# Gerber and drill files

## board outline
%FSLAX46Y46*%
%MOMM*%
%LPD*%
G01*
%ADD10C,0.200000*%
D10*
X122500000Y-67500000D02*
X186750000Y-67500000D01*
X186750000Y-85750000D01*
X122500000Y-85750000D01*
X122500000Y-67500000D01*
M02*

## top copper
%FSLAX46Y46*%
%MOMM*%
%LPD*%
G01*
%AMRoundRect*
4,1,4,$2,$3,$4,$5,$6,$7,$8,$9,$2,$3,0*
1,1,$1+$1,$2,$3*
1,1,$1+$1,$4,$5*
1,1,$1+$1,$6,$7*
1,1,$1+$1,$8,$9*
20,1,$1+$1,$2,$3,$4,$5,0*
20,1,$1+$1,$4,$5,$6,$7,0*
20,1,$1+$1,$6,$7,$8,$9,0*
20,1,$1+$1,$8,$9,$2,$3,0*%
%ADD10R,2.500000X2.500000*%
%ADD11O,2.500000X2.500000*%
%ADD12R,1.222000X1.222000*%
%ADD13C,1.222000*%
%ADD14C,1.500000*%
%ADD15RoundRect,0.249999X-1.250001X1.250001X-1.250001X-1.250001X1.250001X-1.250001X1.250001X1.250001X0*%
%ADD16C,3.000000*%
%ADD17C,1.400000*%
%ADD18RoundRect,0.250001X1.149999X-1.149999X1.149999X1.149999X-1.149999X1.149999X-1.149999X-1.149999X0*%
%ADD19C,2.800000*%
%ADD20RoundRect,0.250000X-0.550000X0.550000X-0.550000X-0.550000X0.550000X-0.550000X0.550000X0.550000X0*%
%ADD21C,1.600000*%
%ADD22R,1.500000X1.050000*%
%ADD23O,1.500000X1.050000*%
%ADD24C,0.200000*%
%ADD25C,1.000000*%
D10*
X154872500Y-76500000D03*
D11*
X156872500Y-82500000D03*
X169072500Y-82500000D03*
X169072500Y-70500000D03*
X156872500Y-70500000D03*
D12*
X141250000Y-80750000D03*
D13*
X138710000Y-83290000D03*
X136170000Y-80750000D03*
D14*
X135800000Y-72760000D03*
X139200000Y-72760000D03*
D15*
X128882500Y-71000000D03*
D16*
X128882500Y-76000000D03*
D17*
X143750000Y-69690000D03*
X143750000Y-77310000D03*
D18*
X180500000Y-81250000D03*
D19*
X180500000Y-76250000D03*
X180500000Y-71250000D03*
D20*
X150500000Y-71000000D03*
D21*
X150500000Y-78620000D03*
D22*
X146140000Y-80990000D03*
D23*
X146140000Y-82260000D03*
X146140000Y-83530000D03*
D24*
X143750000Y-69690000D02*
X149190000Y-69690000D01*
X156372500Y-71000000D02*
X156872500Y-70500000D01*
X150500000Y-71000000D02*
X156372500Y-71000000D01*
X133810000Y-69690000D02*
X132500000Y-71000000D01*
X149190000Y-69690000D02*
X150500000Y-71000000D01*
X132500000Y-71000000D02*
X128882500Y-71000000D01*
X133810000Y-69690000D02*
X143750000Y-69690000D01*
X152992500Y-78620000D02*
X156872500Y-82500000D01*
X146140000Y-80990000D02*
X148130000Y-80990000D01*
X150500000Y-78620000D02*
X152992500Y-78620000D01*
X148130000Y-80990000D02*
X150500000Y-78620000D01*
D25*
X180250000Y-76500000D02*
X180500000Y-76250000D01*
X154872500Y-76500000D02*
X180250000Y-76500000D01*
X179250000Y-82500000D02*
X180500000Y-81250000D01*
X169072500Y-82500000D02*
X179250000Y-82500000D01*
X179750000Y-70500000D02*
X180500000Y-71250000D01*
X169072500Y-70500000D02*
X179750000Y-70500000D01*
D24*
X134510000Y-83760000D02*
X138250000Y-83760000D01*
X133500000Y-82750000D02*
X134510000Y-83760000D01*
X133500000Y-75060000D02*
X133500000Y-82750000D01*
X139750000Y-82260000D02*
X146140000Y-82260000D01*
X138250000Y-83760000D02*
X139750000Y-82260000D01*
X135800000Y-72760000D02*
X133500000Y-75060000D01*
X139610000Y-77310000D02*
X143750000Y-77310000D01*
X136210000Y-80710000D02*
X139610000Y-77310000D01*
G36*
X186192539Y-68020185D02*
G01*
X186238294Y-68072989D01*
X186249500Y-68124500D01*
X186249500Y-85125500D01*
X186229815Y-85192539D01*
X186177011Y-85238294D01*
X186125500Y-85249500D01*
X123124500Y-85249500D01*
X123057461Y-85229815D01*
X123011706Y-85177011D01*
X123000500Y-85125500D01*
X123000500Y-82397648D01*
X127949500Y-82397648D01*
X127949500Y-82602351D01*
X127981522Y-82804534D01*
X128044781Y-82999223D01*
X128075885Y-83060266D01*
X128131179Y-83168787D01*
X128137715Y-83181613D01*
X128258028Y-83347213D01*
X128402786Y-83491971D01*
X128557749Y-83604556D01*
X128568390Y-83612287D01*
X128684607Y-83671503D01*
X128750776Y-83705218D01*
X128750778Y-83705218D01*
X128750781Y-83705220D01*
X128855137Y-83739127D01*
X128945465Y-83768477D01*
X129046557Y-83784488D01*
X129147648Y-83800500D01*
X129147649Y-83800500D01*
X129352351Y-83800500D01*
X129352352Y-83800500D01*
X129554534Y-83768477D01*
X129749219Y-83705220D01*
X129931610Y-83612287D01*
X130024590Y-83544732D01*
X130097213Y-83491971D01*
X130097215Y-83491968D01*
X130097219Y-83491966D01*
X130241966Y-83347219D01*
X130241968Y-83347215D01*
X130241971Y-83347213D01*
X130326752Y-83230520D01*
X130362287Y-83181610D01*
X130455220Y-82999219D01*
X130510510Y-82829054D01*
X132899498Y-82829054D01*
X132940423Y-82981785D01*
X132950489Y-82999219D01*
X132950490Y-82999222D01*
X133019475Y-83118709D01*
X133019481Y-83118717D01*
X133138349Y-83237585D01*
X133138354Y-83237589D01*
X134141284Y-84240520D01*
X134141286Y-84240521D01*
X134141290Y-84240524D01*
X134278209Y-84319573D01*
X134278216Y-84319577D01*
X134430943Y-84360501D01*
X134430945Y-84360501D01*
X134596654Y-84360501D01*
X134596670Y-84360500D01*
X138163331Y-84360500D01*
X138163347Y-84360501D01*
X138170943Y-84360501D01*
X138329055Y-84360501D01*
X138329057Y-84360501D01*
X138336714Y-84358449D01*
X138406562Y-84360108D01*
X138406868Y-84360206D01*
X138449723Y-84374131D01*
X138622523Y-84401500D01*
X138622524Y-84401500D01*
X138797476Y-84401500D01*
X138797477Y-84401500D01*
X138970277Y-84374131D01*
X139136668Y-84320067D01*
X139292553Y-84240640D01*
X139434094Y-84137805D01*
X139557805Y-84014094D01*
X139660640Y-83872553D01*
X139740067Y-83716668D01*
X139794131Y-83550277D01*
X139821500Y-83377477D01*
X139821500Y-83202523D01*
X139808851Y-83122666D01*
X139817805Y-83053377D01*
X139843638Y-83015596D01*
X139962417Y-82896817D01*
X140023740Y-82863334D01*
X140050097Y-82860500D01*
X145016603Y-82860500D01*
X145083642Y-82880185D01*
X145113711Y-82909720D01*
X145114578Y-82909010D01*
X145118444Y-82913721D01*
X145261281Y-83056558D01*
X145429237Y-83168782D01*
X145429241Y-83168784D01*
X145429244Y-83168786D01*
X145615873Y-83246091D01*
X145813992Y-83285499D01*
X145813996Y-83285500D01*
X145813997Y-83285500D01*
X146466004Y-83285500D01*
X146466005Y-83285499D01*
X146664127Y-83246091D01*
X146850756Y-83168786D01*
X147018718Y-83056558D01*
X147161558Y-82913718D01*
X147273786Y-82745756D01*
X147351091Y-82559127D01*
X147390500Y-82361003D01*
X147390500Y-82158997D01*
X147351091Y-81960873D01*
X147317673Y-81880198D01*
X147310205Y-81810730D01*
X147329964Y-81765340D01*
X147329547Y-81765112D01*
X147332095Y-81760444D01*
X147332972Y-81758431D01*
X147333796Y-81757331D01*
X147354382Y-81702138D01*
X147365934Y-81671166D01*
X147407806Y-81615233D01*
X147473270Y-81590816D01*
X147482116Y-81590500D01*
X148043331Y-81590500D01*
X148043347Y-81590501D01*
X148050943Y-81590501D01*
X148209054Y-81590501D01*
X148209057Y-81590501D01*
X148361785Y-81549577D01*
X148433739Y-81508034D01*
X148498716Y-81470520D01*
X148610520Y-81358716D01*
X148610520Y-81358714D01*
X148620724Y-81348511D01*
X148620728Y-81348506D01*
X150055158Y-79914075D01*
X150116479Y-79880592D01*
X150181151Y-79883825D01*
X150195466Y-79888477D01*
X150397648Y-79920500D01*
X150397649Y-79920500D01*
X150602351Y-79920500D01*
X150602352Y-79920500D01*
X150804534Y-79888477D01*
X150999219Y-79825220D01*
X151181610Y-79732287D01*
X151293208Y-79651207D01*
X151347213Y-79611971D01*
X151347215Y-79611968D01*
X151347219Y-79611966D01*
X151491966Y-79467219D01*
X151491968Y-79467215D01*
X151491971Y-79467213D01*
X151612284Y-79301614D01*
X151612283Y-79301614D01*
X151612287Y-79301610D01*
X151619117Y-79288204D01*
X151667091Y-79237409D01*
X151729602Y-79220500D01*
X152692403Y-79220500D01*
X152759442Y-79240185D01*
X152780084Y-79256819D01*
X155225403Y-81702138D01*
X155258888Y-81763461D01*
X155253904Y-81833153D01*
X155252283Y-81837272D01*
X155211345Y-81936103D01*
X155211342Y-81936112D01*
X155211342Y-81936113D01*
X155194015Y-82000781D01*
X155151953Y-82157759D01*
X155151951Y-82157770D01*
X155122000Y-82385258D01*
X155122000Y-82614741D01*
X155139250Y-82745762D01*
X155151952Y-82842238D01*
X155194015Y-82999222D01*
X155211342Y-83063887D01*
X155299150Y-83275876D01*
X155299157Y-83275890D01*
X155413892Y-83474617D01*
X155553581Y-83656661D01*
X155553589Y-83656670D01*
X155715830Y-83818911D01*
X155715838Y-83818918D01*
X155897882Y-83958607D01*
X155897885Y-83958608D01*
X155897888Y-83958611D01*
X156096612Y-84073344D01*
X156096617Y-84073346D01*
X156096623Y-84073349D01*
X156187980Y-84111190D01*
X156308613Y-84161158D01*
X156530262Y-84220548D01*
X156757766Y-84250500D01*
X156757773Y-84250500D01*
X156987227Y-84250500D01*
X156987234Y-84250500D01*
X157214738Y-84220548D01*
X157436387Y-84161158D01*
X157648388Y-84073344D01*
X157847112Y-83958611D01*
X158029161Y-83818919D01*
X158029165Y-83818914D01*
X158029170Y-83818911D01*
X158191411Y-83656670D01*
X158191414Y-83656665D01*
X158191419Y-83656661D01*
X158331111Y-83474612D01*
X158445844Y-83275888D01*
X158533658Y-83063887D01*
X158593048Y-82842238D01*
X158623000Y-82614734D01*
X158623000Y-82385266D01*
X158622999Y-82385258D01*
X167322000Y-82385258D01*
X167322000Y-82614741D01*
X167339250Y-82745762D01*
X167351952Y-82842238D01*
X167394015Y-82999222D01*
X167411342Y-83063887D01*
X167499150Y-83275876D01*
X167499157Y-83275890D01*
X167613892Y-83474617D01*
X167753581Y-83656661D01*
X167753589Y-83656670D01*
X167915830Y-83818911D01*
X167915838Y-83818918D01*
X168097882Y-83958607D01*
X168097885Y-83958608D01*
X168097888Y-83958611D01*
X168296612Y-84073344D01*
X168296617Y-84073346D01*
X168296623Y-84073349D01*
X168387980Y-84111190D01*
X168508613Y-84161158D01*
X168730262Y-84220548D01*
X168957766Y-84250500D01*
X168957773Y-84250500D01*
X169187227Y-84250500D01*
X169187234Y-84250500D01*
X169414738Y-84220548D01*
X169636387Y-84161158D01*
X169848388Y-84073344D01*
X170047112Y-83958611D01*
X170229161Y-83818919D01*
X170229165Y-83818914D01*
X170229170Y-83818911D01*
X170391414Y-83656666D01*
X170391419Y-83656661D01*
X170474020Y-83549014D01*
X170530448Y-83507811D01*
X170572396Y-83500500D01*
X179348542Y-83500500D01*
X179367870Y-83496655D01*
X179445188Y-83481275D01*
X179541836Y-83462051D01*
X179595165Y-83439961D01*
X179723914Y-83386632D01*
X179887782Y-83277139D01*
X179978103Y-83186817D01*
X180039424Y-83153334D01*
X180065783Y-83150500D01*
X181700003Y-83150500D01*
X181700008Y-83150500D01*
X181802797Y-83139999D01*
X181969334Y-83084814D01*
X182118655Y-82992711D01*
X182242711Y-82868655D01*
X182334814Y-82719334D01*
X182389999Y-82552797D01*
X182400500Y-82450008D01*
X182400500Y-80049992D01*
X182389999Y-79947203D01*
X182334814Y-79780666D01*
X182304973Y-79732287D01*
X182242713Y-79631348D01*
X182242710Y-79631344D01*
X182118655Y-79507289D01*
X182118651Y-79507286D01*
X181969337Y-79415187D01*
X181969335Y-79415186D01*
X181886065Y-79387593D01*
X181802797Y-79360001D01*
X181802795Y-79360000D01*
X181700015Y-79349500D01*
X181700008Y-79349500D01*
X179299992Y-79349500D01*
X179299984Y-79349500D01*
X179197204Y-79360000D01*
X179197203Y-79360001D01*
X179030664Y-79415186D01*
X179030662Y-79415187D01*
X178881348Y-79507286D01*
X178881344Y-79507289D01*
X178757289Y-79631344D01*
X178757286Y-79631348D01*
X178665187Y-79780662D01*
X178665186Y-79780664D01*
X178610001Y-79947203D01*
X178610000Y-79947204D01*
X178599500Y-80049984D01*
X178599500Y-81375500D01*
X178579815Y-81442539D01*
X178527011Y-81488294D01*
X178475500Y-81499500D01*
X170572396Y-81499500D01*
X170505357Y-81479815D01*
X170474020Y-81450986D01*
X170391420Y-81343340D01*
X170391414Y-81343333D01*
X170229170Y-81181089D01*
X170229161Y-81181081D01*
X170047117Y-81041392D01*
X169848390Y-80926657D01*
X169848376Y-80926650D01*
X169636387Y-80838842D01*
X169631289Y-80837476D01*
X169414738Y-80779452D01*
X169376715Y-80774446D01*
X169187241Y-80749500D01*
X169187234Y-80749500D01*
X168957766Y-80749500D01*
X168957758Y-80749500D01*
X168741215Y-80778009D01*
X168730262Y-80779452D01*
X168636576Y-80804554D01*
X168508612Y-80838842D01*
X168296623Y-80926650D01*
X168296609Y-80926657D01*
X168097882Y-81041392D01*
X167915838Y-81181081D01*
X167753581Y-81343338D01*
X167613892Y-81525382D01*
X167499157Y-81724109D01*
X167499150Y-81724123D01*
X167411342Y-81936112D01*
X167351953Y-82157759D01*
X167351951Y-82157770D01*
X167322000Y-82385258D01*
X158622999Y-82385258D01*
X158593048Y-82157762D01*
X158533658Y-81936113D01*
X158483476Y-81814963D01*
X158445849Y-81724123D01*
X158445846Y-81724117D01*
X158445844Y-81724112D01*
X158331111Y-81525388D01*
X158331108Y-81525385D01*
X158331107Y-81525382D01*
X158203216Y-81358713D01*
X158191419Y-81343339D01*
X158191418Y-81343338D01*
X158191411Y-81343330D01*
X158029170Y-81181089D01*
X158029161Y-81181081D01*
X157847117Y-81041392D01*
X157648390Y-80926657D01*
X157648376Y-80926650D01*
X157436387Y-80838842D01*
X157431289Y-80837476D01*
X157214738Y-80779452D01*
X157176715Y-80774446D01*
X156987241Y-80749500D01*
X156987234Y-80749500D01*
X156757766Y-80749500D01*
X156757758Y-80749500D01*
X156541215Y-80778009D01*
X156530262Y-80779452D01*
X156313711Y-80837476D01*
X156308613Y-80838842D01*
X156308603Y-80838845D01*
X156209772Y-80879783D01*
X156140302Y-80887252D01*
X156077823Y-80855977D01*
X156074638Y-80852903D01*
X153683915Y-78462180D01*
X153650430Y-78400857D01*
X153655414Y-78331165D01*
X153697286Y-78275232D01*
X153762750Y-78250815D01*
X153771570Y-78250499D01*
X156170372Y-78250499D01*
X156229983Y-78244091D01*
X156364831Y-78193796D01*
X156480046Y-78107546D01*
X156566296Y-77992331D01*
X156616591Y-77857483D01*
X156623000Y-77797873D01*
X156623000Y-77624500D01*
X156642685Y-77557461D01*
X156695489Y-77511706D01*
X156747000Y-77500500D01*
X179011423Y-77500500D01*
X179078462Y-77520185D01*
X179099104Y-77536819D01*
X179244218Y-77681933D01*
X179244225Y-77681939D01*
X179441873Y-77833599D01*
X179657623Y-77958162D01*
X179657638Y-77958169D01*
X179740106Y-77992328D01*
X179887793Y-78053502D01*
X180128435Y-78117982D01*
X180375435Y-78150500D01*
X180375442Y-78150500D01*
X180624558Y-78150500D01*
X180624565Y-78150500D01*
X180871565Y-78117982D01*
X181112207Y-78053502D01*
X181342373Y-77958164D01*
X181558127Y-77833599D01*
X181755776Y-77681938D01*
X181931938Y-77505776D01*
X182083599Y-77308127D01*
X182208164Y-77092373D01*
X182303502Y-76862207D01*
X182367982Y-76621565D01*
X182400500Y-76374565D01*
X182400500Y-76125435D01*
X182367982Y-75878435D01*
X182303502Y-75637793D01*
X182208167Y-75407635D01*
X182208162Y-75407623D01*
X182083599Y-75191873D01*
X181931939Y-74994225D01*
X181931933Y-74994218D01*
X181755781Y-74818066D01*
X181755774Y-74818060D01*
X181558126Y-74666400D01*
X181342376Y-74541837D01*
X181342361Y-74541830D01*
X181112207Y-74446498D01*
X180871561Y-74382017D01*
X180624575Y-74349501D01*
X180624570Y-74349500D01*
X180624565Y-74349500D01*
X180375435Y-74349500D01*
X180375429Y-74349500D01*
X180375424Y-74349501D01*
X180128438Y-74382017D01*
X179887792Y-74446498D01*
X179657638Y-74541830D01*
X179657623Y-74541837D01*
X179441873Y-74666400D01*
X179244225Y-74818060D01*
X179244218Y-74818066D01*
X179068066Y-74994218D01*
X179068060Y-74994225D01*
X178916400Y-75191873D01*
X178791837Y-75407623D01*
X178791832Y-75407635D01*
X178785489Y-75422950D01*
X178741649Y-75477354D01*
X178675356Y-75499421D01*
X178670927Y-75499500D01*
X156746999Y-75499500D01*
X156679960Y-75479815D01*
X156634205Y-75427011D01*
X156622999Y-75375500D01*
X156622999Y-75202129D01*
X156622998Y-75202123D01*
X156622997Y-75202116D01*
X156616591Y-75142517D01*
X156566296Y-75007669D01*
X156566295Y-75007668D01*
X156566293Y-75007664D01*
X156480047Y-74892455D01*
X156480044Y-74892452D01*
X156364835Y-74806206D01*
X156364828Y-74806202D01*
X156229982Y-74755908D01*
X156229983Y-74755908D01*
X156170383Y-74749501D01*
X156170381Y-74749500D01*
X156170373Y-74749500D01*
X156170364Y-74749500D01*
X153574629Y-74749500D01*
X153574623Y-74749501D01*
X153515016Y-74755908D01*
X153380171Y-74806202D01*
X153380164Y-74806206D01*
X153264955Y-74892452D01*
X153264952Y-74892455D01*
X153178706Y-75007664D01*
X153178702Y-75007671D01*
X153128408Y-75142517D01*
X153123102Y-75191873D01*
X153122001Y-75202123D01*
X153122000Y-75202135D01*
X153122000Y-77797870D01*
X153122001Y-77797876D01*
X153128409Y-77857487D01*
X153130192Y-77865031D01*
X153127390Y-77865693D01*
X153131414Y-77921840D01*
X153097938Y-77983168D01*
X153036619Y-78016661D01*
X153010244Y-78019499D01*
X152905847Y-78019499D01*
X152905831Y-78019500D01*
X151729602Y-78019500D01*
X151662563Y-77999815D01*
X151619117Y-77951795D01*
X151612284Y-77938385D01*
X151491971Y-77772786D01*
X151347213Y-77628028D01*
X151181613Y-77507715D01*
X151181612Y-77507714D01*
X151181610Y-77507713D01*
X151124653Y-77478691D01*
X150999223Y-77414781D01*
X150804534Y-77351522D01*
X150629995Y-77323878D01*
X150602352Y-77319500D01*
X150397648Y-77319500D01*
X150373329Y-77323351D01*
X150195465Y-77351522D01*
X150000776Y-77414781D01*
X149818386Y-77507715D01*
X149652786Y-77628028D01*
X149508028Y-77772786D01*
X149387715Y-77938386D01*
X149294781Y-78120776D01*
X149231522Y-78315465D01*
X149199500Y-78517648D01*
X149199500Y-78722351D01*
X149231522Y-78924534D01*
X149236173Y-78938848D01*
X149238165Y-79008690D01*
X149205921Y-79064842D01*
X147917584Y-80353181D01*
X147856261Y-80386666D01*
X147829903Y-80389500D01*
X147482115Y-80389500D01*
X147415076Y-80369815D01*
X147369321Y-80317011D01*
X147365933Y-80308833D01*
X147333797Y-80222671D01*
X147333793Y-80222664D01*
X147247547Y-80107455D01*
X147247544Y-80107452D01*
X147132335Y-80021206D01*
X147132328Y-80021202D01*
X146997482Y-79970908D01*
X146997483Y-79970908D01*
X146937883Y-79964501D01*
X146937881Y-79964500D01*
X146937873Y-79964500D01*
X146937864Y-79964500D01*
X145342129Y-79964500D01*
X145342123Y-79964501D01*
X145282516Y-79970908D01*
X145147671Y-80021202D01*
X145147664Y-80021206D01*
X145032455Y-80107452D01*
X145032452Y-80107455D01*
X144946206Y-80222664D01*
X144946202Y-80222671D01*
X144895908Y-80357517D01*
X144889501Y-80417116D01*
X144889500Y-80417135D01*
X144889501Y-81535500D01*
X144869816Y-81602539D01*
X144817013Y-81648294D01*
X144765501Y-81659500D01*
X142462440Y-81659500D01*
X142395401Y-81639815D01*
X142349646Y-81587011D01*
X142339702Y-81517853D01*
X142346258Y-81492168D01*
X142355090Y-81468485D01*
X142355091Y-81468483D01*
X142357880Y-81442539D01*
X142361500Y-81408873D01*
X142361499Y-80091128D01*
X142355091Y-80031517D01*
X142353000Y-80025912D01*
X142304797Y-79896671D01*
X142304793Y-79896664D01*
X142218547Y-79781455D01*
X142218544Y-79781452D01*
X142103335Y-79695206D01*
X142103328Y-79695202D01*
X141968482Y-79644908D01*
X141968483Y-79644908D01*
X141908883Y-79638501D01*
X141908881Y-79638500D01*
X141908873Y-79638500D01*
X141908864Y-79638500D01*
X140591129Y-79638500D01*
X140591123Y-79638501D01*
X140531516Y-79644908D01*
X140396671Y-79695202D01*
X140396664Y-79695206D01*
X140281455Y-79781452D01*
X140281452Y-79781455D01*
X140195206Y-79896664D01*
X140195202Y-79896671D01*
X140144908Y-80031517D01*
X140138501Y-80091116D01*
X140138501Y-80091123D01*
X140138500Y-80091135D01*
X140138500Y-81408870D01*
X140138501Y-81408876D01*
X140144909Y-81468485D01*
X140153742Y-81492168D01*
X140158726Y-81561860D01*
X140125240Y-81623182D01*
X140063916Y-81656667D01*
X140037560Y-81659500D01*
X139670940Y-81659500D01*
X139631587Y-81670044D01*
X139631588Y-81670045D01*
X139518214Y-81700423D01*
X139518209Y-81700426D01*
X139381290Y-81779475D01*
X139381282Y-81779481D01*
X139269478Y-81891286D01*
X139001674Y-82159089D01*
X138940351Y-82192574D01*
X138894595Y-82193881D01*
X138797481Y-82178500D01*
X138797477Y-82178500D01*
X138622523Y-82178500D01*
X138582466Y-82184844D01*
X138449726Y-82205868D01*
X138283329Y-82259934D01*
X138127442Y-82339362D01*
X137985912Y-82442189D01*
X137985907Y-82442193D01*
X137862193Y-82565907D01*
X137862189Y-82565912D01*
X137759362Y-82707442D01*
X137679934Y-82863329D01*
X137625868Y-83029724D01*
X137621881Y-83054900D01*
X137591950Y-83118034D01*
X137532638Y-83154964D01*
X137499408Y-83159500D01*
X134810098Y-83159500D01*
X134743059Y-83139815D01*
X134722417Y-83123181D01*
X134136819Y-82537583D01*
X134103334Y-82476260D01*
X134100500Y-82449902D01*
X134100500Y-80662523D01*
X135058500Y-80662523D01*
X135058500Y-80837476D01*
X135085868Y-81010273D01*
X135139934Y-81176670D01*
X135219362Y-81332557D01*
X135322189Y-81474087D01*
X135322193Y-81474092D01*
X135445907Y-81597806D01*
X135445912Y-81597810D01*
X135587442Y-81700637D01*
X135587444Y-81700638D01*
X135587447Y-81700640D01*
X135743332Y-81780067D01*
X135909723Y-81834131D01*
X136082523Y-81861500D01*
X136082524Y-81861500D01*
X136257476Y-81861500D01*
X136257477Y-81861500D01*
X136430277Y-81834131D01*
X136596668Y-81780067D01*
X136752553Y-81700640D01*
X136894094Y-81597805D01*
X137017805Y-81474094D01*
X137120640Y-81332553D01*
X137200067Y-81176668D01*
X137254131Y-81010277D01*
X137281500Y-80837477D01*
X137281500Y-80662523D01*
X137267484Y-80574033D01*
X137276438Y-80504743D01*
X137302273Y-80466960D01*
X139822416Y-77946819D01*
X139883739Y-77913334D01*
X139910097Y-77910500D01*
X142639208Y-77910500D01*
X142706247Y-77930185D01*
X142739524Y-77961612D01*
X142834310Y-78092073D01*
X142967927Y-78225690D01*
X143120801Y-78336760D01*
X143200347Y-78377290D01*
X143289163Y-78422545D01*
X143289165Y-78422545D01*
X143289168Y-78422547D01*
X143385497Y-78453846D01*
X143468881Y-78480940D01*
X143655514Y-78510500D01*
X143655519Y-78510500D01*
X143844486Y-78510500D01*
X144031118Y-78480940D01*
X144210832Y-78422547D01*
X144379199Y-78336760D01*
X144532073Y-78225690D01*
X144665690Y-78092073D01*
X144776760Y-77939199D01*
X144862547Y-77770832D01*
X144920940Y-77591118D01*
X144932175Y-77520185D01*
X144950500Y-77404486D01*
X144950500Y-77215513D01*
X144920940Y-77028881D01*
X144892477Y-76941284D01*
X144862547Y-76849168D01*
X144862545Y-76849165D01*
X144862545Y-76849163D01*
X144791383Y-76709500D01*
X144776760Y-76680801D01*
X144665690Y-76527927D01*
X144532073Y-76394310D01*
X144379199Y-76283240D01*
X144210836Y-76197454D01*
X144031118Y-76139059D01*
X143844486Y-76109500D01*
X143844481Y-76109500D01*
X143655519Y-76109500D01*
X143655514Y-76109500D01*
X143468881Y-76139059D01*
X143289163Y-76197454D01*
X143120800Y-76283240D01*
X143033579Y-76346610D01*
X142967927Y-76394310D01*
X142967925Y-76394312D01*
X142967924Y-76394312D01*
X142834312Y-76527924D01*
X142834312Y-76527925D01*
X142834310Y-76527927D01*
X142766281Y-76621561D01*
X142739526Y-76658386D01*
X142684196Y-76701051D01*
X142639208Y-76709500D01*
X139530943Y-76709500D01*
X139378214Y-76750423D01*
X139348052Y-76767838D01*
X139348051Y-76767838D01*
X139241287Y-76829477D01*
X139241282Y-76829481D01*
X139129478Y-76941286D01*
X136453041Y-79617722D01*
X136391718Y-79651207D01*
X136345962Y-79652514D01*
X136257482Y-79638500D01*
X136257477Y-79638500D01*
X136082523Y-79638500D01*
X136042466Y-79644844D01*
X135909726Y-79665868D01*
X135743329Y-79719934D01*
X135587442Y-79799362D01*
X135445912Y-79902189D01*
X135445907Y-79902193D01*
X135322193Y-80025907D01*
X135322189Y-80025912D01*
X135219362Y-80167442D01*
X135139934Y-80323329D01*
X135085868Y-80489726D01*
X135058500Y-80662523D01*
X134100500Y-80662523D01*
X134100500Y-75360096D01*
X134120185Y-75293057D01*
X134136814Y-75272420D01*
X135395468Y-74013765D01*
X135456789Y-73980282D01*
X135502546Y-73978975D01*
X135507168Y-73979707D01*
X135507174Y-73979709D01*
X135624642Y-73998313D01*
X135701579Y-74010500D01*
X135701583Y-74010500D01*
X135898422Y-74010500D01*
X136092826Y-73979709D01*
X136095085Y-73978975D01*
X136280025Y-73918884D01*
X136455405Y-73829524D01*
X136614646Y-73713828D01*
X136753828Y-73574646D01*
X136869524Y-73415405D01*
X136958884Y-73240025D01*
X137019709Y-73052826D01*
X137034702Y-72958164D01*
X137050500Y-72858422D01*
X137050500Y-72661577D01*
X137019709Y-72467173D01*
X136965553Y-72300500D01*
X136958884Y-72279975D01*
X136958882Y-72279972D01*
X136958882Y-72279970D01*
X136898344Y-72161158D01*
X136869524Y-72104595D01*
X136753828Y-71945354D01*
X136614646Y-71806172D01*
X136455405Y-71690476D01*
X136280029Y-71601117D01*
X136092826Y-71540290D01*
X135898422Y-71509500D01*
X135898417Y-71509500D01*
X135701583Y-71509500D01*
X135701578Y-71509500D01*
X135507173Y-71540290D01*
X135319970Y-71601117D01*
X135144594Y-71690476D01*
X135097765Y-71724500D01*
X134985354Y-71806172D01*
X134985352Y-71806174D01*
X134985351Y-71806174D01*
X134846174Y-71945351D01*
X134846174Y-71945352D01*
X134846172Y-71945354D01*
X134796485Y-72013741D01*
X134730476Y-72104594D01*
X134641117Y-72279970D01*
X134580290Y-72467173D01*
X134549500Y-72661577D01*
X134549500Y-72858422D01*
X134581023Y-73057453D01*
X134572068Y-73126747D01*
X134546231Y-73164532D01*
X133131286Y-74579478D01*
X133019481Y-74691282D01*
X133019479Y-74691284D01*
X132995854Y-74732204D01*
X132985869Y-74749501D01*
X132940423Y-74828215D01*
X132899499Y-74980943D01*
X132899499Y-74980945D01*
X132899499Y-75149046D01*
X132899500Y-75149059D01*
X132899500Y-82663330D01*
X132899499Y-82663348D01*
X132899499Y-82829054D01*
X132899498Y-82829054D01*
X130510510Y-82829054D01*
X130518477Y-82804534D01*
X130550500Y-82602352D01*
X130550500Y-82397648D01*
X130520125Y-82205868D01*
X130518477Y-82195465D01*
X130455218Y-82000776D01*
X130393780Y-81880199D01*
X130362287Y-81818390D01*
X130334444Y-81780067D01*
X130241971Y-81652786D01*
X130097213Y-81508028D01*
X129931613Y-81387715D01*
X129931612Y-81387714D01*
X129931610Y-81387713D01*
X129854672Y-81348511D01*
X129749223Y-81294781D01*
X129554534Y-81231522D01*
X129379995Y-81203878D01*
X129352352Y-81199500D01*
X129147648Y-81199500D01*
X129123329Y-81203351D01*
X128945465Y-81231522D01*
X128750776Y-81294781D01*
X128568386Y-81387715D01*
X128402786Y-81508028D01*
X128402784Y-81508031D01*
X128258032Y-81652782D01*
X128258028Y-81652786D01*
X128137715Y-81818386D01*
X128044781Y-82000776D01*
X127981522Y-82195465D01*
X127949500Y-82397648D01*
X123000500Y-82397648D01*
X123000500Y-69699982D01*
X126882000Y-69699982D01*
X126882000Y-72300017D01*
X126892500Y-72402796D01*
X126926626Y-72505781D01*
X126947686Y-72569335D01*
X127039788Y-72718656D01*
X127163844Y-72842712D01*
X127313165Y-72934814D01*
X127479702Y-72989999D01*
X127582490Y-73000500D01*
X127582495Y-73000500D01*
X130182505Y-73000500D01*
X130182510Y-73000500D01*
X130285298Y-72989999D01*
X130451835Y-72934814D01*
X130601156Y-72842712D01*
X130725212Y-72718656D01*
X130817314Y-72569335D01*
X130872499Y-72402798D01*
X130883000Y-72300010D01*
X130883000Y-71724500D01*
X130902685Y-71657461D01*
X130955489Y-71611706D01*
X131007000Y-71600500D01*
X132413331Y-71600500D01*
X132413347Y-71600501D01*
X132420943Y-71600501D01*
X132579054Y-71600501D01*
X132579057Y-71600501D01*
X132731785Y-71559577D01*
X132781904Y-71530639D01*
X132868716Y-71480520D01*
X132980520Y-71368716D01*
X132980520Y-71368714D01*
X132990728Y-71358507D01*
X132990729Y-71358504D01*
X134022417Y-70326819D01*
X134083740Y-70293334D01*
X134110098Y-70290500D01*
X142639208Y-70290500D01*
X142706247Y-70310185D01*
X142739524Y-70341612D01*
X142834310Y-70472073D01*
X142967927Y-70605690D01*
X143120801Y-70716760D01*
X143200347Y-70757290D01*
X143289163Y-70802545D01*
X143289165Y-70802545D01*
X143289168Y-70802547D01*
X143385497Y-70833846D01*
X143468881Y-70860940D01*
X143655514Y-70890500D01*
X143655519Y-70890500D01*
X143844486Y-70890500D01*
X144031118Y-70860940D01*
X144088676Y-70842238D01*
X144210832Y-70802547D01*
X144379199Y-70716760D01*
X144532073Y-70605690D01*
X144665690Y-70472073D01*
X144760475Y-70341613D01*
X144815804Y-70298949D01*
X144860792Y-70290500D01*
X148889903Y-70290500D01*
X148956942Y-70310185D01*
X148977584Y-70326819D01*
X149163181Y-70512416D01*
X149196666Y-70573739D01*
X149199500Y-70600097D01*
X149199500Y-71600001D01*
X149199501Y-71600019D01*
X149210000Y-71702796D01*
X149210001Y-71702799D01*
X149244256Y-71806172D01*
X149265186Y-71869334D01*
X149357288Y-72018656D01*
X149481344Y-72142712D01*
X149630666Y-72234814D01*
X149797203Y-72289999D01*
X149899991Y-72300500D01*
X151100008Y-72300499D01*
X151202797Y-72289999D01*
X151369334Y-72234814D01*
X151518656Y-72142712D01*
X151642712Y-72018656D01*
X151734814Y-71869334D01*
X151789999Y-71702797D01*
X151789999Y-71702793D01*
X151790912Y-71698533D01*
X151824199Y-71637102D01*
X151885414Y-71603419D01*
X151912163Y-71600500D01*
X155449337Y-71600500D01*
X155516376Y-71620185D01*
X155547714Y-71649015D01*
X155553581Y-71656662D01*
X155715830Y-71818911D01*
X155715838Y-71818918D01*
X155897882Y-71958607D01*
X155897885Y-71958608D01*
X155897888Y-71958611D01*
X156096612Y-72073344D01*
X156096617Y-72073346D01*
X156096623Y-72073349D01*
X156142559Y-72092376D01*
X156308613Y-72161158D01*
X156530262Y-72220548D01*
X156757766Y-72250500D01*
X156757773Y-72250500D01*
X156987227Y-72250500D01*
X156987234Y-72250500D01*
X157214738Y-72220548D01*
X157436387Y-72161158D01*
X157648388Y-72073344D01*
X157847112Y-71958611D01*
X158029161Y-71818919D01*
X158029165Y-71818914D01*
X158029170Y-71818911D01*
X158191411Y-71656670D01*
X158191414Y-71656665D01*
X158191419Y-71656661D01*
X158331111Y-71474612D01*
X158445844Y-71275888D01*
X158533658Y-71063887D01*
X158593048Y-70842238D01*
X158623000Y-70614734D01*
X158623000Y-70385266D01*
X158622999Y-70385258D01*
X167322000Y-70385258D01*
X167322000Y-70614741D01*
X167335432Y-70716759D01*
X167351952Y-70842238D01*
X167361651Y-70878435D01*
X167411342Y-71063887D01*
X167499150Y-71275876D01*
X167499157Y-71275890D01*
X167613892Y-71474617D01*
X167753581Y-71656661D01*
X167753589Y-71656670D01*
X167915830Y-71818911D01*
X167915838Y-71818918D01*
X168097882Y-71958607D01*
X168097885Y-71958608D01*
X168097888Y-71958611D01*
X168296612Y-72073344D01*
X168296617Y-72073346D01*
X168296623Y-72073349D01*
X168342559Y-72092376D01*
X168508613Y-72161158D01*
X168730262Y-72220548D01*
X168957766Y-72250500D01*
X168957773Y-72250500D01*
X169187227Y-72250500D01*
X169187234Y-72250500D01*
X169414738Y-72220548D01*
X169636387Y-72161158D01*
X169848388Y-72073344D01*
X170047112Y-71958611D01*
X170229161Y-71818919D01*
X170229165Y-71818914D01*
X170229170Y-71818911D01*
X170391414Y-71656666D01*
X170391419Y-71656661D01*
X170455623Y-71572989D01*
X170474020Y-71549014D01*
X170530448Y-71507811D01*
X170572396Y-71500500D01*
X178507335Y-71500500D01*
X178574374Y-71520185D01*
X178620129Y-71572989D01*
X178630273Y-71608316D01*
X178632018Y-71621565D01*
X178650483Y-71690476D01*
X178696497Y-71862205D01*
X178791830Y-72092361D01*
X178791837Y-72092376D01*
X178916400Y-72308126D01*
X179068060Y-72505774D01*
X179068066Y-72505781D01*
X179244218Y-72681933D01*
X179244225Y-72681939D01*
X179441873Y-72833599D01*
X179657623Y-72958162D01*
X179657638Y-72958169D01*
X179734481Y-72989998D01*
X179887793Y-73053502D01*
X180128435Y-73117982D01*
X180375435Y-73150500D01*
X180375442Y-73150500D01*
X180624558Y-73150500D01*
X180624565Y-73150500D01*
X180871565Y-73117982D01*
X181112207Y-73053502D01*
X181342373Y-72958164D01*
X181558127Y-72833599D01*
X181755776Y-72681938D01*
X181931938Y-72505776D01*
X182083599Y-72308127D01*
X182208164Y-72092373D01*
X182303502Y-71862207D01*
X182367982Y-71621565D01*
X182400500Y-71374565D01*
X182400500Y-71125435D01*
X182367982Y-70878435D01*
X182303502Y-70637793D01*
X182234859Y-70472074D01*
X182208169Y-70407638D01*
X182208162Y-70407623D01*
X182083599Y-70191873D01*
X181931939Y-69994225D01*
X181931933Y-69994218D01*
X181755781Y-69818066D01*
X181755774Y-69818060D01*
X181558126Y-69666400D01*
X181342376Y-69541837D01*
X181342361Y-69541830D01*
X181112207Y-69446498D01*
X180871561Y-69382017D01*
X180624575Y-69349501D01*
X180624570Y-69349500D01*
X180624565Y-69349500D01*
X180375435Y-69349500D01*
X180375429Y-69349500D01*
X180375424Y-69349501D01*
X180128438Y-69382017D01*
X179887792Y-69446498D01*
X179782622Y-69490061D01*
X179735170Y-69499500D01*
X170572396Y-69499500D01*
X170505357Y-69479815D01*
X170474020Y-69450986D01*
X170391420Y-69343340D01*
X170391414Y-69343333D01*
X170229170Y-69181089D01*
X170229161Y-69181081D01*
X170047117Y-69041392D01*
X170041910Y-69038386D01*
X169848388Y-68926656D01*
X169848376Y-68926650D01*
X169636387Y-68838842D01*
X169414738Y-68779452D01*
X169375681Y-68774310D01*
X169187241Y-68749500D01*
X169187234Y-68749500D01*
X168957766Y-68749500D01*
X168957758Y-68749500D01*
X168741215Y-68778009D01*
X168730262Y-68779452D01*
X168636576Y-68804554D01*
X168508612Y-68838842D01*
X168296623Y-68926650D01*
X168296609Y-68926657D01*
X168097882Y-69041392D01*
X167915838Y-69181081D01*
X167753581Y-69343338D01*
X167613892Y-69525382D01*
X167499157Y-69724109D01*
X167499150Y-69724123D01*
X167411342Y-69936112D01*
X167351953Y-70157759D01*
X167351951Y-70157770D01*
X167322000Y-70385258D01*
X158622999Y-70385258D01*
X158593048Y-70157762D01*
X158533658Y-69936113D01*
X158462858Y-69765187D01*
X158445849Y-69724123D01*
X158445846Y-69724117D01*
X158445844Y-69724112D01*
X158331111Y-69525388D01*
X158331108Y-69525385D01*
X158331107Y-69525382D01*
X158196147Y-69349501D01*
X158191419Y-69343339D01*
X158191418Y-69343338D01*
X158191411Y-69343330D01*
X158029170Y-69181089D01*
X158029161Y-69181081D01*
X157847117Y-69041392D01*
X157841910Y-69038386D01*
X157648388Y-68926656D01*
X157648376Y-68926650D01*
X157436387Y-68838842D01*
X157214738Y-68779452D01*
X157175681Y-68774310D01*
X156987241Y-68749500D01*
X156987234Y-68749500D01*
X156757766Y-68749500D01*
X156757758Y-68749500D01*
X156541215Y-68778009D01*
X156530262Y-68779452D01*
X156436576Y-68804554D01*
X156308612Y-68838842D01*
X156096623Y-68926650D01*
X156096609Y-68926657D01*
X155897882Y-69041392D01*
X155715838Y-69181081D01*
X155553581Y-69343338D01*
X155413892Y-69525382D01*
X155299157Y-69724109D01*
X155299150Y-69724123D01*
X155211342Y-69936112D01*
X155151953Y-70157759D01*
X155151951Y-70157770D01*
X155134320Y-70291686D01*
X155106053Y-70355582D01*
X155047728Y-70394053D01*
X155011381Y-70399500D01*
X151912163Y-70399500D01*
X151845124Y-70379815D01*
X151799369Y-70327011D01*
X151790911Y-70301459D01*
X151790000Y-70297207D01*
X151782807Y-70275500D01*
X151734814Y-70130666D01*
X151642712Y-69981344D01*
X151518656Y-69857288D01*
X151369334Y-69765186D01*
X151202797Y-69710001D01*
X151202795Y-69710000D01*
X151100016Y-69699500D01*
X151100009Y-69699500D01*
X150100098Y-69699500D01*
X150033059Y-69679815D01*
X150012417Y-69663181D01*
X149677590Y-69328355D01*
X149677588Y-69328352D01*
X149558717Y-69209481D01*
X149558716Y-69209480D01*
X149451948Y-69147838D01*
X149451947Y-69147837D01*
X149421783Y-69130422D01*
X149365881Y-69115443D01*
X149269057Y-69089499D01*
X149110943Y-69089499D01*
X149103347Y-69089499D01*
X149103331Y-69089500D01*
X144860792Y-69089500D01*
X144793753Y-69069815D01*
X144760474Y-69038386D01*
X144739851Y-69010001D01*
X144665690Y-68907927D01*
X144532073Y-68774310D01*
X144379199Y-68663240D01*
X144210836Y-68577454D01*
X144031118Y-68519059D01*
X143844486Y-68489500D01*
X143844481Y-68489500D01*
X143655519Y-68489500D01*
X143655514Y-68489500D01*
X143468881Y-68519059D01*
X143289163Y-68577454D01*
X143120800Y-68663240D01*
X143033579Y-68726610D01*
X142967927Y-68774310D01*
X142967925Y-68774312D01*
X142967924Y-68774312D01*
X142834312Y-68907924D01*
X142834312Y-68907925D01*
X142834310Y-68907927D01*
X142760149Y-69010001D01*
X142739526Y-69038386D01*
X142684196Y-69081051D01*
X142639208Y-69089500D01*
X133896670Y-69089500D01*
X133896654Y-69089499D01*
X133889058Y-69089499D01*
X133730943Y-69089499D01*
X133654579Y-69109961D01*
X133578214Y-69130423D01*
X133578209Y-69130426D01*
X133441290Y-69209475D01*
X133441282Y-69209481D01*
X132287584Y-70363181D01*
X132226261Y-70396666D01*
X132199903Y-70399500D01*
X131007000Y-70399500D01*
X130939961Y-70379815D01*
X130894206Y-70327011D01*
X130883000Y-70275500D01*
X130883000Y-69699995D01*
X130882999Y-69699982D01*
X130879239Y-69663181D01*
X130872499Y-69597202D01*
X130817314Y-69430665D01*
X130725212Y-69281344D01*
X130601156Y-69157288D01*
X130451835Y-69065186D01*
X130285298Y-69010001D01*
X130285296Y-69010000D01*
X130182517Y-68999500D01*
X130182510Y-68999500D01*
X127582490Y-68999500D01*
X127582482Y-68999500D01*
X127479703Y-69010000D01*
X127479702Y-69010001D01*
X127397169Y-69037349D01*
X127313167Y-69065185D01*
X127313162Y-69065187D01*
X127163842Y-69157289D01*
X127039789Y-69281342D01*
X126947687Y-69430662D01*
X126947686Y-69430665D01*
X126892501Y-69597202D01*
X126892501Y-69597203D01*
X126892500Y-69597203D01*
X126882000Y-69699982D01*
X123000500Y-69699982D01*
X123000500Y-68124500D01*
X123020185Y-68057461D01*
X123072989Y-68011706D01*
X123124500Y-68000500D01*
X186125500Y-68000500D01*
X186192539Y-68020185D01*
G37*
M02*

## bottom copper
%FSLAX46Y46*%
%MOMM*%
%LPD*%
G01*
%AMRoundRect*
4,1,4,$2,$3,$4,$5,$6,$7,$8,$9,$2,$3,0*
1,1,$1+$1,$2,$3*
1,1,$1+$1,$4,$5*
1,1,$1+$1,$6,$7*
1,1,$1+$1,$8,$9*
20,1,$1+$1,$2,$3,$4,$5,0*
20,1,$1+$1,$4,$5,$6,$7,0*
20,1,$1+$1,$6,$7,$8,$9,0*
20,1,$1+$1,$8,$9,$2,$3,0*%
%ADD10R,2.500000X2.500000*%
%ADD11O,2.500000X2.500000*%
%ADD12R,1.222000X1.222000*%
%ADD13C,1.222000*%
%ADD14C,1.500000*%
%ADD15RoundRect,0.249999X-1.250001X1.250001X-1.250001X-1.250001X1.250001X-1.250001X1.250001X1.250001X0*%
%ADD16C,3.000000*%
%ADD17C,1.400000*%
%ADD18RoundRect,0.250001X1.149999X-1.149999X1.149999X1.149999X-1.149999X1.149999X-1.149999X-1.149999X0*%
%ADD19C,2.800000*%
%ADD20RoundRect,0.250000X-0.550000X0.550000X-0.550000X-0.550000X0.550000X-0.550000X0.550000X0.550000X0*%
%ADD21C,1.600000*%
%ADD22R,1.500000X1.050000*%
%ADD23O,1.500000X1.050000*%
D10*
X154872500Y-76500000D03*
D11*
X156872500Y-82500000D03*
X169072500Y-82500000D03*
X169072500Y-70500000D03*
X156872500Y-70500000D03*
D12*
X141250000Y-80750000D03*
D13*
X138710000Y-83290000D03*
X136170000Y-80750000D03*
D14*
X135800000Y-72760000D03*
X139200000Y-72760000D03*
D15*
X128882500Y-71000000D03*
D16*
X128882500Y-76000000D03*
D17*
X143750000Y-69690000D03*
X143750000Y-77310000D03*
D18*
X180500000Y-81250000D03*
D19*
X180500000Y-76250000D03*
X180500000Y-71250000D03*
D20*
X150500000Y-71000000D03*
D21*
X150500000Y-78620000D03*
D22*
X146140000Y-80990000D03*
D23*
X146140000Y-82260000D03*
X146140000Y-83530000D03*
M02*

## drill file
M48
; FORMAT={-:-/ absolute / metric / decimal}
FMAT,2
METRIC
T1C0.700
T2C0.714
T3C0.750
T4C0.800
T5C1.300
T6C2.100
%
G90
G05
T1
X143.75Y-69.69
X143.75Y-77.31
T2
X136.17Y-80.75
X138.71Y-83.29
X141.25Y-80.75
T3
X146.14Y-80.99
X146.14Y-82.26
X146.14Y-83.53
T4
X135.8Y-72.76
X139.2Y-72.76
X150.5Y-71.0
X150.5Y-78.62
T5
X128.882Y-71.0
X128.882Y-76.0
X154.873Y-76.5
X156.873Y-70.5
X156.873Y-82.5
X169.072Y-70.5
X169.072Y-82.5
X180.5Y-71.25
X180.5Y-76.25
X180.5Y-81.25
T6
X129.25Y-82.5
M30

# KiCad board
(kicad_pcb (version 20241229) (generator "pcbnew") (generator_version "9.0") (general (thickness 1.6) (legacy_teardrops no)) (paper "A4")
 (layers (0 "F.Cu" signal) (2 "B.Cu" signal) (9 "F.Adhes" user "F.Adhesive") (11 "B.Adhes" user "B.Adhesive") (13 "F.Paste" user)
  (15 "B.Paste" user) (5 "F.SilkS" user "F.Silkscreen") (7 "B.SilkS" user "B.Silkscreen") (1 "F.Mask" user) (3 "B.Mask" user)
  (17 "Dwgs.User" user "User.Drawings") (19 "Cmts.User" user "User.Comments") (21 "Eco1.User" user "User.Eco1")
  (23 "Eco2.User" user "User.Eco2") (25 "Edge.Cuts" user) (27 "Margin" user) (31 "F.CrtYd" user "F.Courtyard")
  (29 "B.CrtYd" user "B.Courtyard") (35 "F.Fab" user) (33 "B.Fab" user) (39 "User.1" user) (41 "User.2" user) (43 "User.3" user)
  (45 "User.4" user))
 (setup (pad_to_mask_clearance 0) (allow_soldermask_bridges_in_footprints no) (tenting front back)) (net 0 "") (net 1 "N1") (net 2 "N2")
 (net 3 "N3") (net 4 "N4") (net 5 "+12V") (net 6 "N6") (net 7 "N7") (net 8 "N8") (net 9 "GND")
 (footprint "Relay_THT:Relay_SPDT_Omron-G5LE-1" (layer "F.Cu") (at 154.8725 76.5 90)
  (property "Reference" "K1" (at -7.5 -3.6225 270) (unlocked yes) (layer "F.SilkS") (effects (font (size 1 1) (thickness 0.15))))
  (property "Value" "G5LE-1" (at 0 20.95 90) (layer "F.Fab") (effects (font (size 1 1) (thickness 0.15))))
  (pad "1" thru_hole rect (at 0 0 90) (size 2.5 2.5) (drill 1.3) (layers "*.Cu" "*.Mask") (remove_unused_layers no) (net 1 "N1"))
  (pad "2" thru_hole oval (at -6 2 90) (size 2.5 2.5) (drill 1.3) (layers "*.Cu" "*.Mask") (remove_unused_layers no) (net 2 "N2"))
  (pad "3" thru_hole oval (at -6 14.2 90) (size 2.5 2.5) (drill 1.3) (layers "*.Cu" "*.Mask") (remove_unused_layers no) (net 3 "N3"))
  (pad "4" thru_hole oval (at 6 14.2 90) (size 2.5 2.5) (drill 1.3) (layers "*.Cu" "*.Mask") (remove_unused_layers no) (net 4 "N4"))
  (pad "5" thru_hole oval (at 6 2 90) (size 2.5 2.5) (drill 1.3) (layers "*.Cu" "*.Mask") (remove_unused_layers no) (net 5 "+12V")))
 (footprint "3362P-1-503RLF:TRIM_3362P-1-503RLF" (layer "F.Cu") (at 138.71 80.75 180)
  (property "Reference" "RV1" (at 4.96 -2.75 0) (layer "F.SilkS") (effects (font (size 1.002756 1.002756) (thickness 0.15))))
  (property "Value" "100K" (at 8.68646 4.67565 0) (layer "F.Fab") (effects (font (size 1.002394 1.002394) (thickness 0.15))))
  (pad "1" thru_hole rect (at -2.54 0 180) (size 1.222 1.222) (drill 0.714) (layers "*.Cu" "*.Mask") (remove_unused_layers no) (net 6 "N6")
   (solder_mask_margin 0.102))
  (pad "2" thru_hole circle (at 0 -2.54 180) (size 1.222 1.222) (drill 0.714) (layers "*.Cu" "*.Mask") (remove_unused_layers no)
   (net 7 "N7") (solder_mask_margin 0.102))
  (pad "3" thru_hole circle (at 2.54 0 180) (size 1.222 1.222) (drill 0.714) (layers "*.Cu" "*.Mask") (remove_unused_layers no) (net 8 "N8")
   (solder_mask_margin 0.102)))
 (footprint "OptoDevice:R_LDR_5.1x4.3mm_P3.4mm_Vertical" (layer "F.Cu") (at 135.8 72.76)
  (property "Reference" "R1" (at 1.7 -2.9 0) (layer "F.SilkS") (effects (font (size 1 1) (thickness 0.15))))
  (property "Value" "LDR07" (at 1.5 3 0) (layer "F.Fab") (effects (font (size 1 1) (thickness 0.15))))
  (pad "1" thru_hole circle (at 0 0) (size 1.5 1.5) (drill 0.8) (layers "*.Cu" "*.Mask") (remove_unused_layers no) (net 7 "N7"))
  (pad "2" thru_hole circle (at 3.4 0) (size 1.5 1.5) (drill 0.8) (layers "*.Cu" "*.Mask") (remove_unused_layers no) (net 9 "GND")))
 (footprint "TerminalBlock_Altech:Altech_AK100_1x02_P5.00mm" (layer "F.Cu") (at 128.8825 71 -90)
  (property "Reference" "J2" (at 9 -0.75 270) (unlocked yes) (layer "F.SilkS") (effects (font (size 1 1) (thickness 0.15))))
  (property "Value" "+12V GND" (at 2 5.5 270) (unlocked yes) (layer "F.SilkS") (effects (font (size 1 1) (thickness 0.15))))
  (pad "1" thru_hole roundrect (at 0 0 270) (size 3 3) (drill 1.3) (layers "*.Cu" "*.Mask") (remove_unused_layers no)
   (roundrect_rratio 0.083333) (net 5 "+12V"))
  (pad "2" thru_hole circle (at 5 0 270) (size 3 3) (drill 1.3) (layers "*.Cu" "*.Mask") (remove_unused_layers no) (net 9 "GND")))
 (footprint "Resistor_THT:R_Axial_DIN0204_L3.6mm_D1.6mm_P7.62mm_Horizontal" (layer "F.Cu") (at 143.75 69.69 -90)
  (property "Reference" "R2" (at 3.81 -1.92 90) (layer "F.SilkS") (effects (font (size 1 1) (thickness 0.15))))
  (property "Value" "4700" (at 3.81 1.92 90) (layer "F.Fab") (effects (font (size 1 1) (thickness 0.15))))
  (pad "1" thru_hole circle (at 0 0 270) (size 1.4 1.4) (drill 0.7) (layers "*.Cu" "*.Mask") (remove_unused_layers no) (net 5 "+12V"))
  (pad "2" thru_hole circle (at 7.62 0 270) (size 1.4 1.4) (drill 0.7) (layers "*.Cu" "*.Mask") (remove_unused_layers no) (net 8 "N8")))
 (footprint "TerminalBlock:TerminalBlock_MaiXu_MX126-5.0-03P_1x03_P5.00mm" (layer "F.Cu") (at 180.5 81.25 90)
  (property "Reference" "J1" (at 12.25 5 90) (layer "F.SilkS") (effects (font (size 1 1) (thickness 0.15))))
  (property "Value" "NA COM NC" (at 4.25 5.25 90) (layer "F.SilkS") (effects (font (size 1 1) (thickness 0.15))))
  (pad "1" thru_hole roundrect (at 0 0 90) (size 2.8 2.8) (drill 1.3) (layers "*.Cu" "*.Mask") (remove_unused_layers no)
   (roundrect_rratio 0.089286) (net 3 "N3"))
  (pad "2" thru_hole circle (at 5 0 90) (size 2.8 2.8) (drill 1.3) (layers "*.Cu" "*.Mask") (remove_unused_layers no) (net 1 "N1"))
  (pad "3" thru_hole circle (at 10 0 90) (size 2.8 2.8) (drill 1.3) (layers "*.Cu" "*.Mask") (remove_unused_layers no) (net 4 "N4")))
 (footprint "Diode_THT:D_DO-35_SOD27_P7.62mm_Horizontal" (layer "F.Cu") (at 150.5 71 -90)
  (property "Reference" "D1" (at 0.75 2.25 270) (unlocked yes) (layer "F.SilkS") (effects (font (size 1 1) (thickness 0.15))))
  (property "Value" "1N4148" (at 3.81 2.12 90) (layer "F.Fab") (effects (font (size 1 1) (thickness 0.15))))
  (pad "1" thru_hole roundrect (at 0 0 270) (size 1.6 1.6) (drill 0.8) (layers "*.Cu" "*.Mask") (remove_unused_layers no)
   (roundrect_rratio 0.15625) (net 5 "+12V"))
  (pad "2" thru_hole circle (at 7.62 0 270) (size 1.6 1.6) (drill 0.8) (layers "*.Cu" "*.Mask") (remove_unused_layers no) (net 2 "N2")))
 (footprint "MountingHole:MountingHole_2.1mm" (layer "F.Cu") (at 129.25 82.5)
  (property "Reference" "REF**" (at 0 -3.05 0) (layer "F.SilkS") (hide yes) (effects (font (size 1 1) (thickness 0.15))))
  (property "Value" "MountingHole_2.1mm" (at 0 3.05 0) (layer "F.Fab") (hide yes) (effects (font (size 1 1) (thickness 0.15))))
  (pad "" np_thru_hole circle (at 0 0) (size 2.1 2.1) (drill 2.1) (layers "*.Cu" "*.Mask")))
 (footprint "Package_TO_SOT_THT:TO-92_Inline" (layer "F.Cu") (at 146.14 80.99 -90)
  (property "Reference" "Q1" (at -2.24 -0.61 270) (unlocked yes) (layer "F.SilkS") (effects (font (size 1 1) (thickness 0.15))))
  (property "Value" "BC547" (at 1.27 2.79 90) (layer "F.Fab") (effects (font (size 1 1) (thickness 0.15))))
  (pad "1" thru_hole rect (at 0 0 270) (size 1.05 1.5) (drill 0.75) (layers "*.Cu" "*.Mask") (remove_unused_layers no) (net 2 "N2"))
  (pad "2" thru_hole oval (at 1.27 0 270) (size 1.05 1.5) (drill 0.75) (layers "*.Cu" "*.Mask") (remove_unused_layers no) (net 7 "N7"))
  (pad "3" thru_hole oval (at 2.54 0 270) (size 1.05 1.5) (drill 0.75) (layers "*.Cu" "*.Mask") (remove_unused_layers no) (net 9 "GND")))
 (gr_rect (start 122.5 67.5) (end 186.75 85.75) (stroke (width 0.2) (type solid)) (fill no) (layer "Edge.Cuts"))
 (segment (start 143.75 69.69) (end 149.19 69.69) (width 0.2) (layer "F.Cu") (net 5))
 (segment (start 156.3725 71) (end 156.8725 70.5) (width 0.2) (layer "F.Cu") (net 5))
 (segment (start 150.5 71) (end 156.3725 71) (width 0.2) (layer "F.Cu") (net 5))
 (segment (start 133.81 69.69) (end 132.5 71) (width 0.2) (layer "F.Cu") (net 5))
 (segment (start 149.19 69.69) (end 150.5 71) (width 0.2) (layer "F.Cu") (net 5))
 (segment (start 132.5 71) (end 128.8825 71) (width 0.2) (layer "F.Cu") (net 5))
 (segment (start 133.81 69.69) (end 143.75 69.69) (width 0.2) (layer "F.Cu") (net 5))
 (segment (start 152.9925 78.62) (end 156.8725 82.5) (width 0.2) (layer "F.Cu") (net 2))
 (segment (start 146.14 80.99) (end 148.13 80.99) (width 0.2) (layer "F.Cu") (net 2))
 (segment (start 150.5 78.62) (end 152.9925 78.62) (width 0.2) (layer "F.Cu") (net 2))
 (segment (start 148.13 80.99) (end 150.5 78.62) (width 0.2) (layer "F.Cu") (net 2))
 (segment (start 180.25 76.5) (end 180.5 76.25) (width 1) (layer "F.Cu") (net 1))
 (segment (start 154.8725 76.5) (end 180.25 76.5) (width 1) (layer "F.Cu") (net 1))
 (segment (start 179.25 82.5) (end 180.5 81.25) (width 1) (layer "F.Cu") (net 3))
 (segment (start 169.0725 82.5) (end 179.25 82.5) (width 1) (layer "F.Cu") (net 3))
 (segment (start 179.75 70.5) (end 180.5 71.25) (width 1) (layer "F.Cu") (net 4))
 (segment (start 169.0725 70.5) (end 179.75 70.5) (width 1) (layer "F.Cu") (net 4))
 (segment (start 134.51 83.76) (end 138.25 83.76) (width 0.2) (layer "F.Cu") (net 7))
 (segment (start 133.5 82.75) (end 134.51 83.76) (width 0.2) (layer "F.Cu") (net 7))
 (segment (start 133.5 75.06) (end 133.5 82.75) (width 0.2) (layer "F.Cu") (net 7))
 (segment (start 139.75 82.26) (end 146.14 82.26) (width 0.2) (layer "F.Cu") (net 7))
 (segment (start 138.25 83.76) (end 139.75 82.26) (width 0.2) (layer "F.Cu") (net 7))
 (segment (start 135.8 72.76) (end 133.5 75.06) (width 0.2) (layer "F.Cu") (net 7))
 (segment (start 139.61 77.31) (end 143.75 77.31) (width 0.2) (layer "F.Cu") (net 8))
 (segment (start 136.21 80.71) (end 139.61 77.31) (width 0.2) (layer "F.Cu") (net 8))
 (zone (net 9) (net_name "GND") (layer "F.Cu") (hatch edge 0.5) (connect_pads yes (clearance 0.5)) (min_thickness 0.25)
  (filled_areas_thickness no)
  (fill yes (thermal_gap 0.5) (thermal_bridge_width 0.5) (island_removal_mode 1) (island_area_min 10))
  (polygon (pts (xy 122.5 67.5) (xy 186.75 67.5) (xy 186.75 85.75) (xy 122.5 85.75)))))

